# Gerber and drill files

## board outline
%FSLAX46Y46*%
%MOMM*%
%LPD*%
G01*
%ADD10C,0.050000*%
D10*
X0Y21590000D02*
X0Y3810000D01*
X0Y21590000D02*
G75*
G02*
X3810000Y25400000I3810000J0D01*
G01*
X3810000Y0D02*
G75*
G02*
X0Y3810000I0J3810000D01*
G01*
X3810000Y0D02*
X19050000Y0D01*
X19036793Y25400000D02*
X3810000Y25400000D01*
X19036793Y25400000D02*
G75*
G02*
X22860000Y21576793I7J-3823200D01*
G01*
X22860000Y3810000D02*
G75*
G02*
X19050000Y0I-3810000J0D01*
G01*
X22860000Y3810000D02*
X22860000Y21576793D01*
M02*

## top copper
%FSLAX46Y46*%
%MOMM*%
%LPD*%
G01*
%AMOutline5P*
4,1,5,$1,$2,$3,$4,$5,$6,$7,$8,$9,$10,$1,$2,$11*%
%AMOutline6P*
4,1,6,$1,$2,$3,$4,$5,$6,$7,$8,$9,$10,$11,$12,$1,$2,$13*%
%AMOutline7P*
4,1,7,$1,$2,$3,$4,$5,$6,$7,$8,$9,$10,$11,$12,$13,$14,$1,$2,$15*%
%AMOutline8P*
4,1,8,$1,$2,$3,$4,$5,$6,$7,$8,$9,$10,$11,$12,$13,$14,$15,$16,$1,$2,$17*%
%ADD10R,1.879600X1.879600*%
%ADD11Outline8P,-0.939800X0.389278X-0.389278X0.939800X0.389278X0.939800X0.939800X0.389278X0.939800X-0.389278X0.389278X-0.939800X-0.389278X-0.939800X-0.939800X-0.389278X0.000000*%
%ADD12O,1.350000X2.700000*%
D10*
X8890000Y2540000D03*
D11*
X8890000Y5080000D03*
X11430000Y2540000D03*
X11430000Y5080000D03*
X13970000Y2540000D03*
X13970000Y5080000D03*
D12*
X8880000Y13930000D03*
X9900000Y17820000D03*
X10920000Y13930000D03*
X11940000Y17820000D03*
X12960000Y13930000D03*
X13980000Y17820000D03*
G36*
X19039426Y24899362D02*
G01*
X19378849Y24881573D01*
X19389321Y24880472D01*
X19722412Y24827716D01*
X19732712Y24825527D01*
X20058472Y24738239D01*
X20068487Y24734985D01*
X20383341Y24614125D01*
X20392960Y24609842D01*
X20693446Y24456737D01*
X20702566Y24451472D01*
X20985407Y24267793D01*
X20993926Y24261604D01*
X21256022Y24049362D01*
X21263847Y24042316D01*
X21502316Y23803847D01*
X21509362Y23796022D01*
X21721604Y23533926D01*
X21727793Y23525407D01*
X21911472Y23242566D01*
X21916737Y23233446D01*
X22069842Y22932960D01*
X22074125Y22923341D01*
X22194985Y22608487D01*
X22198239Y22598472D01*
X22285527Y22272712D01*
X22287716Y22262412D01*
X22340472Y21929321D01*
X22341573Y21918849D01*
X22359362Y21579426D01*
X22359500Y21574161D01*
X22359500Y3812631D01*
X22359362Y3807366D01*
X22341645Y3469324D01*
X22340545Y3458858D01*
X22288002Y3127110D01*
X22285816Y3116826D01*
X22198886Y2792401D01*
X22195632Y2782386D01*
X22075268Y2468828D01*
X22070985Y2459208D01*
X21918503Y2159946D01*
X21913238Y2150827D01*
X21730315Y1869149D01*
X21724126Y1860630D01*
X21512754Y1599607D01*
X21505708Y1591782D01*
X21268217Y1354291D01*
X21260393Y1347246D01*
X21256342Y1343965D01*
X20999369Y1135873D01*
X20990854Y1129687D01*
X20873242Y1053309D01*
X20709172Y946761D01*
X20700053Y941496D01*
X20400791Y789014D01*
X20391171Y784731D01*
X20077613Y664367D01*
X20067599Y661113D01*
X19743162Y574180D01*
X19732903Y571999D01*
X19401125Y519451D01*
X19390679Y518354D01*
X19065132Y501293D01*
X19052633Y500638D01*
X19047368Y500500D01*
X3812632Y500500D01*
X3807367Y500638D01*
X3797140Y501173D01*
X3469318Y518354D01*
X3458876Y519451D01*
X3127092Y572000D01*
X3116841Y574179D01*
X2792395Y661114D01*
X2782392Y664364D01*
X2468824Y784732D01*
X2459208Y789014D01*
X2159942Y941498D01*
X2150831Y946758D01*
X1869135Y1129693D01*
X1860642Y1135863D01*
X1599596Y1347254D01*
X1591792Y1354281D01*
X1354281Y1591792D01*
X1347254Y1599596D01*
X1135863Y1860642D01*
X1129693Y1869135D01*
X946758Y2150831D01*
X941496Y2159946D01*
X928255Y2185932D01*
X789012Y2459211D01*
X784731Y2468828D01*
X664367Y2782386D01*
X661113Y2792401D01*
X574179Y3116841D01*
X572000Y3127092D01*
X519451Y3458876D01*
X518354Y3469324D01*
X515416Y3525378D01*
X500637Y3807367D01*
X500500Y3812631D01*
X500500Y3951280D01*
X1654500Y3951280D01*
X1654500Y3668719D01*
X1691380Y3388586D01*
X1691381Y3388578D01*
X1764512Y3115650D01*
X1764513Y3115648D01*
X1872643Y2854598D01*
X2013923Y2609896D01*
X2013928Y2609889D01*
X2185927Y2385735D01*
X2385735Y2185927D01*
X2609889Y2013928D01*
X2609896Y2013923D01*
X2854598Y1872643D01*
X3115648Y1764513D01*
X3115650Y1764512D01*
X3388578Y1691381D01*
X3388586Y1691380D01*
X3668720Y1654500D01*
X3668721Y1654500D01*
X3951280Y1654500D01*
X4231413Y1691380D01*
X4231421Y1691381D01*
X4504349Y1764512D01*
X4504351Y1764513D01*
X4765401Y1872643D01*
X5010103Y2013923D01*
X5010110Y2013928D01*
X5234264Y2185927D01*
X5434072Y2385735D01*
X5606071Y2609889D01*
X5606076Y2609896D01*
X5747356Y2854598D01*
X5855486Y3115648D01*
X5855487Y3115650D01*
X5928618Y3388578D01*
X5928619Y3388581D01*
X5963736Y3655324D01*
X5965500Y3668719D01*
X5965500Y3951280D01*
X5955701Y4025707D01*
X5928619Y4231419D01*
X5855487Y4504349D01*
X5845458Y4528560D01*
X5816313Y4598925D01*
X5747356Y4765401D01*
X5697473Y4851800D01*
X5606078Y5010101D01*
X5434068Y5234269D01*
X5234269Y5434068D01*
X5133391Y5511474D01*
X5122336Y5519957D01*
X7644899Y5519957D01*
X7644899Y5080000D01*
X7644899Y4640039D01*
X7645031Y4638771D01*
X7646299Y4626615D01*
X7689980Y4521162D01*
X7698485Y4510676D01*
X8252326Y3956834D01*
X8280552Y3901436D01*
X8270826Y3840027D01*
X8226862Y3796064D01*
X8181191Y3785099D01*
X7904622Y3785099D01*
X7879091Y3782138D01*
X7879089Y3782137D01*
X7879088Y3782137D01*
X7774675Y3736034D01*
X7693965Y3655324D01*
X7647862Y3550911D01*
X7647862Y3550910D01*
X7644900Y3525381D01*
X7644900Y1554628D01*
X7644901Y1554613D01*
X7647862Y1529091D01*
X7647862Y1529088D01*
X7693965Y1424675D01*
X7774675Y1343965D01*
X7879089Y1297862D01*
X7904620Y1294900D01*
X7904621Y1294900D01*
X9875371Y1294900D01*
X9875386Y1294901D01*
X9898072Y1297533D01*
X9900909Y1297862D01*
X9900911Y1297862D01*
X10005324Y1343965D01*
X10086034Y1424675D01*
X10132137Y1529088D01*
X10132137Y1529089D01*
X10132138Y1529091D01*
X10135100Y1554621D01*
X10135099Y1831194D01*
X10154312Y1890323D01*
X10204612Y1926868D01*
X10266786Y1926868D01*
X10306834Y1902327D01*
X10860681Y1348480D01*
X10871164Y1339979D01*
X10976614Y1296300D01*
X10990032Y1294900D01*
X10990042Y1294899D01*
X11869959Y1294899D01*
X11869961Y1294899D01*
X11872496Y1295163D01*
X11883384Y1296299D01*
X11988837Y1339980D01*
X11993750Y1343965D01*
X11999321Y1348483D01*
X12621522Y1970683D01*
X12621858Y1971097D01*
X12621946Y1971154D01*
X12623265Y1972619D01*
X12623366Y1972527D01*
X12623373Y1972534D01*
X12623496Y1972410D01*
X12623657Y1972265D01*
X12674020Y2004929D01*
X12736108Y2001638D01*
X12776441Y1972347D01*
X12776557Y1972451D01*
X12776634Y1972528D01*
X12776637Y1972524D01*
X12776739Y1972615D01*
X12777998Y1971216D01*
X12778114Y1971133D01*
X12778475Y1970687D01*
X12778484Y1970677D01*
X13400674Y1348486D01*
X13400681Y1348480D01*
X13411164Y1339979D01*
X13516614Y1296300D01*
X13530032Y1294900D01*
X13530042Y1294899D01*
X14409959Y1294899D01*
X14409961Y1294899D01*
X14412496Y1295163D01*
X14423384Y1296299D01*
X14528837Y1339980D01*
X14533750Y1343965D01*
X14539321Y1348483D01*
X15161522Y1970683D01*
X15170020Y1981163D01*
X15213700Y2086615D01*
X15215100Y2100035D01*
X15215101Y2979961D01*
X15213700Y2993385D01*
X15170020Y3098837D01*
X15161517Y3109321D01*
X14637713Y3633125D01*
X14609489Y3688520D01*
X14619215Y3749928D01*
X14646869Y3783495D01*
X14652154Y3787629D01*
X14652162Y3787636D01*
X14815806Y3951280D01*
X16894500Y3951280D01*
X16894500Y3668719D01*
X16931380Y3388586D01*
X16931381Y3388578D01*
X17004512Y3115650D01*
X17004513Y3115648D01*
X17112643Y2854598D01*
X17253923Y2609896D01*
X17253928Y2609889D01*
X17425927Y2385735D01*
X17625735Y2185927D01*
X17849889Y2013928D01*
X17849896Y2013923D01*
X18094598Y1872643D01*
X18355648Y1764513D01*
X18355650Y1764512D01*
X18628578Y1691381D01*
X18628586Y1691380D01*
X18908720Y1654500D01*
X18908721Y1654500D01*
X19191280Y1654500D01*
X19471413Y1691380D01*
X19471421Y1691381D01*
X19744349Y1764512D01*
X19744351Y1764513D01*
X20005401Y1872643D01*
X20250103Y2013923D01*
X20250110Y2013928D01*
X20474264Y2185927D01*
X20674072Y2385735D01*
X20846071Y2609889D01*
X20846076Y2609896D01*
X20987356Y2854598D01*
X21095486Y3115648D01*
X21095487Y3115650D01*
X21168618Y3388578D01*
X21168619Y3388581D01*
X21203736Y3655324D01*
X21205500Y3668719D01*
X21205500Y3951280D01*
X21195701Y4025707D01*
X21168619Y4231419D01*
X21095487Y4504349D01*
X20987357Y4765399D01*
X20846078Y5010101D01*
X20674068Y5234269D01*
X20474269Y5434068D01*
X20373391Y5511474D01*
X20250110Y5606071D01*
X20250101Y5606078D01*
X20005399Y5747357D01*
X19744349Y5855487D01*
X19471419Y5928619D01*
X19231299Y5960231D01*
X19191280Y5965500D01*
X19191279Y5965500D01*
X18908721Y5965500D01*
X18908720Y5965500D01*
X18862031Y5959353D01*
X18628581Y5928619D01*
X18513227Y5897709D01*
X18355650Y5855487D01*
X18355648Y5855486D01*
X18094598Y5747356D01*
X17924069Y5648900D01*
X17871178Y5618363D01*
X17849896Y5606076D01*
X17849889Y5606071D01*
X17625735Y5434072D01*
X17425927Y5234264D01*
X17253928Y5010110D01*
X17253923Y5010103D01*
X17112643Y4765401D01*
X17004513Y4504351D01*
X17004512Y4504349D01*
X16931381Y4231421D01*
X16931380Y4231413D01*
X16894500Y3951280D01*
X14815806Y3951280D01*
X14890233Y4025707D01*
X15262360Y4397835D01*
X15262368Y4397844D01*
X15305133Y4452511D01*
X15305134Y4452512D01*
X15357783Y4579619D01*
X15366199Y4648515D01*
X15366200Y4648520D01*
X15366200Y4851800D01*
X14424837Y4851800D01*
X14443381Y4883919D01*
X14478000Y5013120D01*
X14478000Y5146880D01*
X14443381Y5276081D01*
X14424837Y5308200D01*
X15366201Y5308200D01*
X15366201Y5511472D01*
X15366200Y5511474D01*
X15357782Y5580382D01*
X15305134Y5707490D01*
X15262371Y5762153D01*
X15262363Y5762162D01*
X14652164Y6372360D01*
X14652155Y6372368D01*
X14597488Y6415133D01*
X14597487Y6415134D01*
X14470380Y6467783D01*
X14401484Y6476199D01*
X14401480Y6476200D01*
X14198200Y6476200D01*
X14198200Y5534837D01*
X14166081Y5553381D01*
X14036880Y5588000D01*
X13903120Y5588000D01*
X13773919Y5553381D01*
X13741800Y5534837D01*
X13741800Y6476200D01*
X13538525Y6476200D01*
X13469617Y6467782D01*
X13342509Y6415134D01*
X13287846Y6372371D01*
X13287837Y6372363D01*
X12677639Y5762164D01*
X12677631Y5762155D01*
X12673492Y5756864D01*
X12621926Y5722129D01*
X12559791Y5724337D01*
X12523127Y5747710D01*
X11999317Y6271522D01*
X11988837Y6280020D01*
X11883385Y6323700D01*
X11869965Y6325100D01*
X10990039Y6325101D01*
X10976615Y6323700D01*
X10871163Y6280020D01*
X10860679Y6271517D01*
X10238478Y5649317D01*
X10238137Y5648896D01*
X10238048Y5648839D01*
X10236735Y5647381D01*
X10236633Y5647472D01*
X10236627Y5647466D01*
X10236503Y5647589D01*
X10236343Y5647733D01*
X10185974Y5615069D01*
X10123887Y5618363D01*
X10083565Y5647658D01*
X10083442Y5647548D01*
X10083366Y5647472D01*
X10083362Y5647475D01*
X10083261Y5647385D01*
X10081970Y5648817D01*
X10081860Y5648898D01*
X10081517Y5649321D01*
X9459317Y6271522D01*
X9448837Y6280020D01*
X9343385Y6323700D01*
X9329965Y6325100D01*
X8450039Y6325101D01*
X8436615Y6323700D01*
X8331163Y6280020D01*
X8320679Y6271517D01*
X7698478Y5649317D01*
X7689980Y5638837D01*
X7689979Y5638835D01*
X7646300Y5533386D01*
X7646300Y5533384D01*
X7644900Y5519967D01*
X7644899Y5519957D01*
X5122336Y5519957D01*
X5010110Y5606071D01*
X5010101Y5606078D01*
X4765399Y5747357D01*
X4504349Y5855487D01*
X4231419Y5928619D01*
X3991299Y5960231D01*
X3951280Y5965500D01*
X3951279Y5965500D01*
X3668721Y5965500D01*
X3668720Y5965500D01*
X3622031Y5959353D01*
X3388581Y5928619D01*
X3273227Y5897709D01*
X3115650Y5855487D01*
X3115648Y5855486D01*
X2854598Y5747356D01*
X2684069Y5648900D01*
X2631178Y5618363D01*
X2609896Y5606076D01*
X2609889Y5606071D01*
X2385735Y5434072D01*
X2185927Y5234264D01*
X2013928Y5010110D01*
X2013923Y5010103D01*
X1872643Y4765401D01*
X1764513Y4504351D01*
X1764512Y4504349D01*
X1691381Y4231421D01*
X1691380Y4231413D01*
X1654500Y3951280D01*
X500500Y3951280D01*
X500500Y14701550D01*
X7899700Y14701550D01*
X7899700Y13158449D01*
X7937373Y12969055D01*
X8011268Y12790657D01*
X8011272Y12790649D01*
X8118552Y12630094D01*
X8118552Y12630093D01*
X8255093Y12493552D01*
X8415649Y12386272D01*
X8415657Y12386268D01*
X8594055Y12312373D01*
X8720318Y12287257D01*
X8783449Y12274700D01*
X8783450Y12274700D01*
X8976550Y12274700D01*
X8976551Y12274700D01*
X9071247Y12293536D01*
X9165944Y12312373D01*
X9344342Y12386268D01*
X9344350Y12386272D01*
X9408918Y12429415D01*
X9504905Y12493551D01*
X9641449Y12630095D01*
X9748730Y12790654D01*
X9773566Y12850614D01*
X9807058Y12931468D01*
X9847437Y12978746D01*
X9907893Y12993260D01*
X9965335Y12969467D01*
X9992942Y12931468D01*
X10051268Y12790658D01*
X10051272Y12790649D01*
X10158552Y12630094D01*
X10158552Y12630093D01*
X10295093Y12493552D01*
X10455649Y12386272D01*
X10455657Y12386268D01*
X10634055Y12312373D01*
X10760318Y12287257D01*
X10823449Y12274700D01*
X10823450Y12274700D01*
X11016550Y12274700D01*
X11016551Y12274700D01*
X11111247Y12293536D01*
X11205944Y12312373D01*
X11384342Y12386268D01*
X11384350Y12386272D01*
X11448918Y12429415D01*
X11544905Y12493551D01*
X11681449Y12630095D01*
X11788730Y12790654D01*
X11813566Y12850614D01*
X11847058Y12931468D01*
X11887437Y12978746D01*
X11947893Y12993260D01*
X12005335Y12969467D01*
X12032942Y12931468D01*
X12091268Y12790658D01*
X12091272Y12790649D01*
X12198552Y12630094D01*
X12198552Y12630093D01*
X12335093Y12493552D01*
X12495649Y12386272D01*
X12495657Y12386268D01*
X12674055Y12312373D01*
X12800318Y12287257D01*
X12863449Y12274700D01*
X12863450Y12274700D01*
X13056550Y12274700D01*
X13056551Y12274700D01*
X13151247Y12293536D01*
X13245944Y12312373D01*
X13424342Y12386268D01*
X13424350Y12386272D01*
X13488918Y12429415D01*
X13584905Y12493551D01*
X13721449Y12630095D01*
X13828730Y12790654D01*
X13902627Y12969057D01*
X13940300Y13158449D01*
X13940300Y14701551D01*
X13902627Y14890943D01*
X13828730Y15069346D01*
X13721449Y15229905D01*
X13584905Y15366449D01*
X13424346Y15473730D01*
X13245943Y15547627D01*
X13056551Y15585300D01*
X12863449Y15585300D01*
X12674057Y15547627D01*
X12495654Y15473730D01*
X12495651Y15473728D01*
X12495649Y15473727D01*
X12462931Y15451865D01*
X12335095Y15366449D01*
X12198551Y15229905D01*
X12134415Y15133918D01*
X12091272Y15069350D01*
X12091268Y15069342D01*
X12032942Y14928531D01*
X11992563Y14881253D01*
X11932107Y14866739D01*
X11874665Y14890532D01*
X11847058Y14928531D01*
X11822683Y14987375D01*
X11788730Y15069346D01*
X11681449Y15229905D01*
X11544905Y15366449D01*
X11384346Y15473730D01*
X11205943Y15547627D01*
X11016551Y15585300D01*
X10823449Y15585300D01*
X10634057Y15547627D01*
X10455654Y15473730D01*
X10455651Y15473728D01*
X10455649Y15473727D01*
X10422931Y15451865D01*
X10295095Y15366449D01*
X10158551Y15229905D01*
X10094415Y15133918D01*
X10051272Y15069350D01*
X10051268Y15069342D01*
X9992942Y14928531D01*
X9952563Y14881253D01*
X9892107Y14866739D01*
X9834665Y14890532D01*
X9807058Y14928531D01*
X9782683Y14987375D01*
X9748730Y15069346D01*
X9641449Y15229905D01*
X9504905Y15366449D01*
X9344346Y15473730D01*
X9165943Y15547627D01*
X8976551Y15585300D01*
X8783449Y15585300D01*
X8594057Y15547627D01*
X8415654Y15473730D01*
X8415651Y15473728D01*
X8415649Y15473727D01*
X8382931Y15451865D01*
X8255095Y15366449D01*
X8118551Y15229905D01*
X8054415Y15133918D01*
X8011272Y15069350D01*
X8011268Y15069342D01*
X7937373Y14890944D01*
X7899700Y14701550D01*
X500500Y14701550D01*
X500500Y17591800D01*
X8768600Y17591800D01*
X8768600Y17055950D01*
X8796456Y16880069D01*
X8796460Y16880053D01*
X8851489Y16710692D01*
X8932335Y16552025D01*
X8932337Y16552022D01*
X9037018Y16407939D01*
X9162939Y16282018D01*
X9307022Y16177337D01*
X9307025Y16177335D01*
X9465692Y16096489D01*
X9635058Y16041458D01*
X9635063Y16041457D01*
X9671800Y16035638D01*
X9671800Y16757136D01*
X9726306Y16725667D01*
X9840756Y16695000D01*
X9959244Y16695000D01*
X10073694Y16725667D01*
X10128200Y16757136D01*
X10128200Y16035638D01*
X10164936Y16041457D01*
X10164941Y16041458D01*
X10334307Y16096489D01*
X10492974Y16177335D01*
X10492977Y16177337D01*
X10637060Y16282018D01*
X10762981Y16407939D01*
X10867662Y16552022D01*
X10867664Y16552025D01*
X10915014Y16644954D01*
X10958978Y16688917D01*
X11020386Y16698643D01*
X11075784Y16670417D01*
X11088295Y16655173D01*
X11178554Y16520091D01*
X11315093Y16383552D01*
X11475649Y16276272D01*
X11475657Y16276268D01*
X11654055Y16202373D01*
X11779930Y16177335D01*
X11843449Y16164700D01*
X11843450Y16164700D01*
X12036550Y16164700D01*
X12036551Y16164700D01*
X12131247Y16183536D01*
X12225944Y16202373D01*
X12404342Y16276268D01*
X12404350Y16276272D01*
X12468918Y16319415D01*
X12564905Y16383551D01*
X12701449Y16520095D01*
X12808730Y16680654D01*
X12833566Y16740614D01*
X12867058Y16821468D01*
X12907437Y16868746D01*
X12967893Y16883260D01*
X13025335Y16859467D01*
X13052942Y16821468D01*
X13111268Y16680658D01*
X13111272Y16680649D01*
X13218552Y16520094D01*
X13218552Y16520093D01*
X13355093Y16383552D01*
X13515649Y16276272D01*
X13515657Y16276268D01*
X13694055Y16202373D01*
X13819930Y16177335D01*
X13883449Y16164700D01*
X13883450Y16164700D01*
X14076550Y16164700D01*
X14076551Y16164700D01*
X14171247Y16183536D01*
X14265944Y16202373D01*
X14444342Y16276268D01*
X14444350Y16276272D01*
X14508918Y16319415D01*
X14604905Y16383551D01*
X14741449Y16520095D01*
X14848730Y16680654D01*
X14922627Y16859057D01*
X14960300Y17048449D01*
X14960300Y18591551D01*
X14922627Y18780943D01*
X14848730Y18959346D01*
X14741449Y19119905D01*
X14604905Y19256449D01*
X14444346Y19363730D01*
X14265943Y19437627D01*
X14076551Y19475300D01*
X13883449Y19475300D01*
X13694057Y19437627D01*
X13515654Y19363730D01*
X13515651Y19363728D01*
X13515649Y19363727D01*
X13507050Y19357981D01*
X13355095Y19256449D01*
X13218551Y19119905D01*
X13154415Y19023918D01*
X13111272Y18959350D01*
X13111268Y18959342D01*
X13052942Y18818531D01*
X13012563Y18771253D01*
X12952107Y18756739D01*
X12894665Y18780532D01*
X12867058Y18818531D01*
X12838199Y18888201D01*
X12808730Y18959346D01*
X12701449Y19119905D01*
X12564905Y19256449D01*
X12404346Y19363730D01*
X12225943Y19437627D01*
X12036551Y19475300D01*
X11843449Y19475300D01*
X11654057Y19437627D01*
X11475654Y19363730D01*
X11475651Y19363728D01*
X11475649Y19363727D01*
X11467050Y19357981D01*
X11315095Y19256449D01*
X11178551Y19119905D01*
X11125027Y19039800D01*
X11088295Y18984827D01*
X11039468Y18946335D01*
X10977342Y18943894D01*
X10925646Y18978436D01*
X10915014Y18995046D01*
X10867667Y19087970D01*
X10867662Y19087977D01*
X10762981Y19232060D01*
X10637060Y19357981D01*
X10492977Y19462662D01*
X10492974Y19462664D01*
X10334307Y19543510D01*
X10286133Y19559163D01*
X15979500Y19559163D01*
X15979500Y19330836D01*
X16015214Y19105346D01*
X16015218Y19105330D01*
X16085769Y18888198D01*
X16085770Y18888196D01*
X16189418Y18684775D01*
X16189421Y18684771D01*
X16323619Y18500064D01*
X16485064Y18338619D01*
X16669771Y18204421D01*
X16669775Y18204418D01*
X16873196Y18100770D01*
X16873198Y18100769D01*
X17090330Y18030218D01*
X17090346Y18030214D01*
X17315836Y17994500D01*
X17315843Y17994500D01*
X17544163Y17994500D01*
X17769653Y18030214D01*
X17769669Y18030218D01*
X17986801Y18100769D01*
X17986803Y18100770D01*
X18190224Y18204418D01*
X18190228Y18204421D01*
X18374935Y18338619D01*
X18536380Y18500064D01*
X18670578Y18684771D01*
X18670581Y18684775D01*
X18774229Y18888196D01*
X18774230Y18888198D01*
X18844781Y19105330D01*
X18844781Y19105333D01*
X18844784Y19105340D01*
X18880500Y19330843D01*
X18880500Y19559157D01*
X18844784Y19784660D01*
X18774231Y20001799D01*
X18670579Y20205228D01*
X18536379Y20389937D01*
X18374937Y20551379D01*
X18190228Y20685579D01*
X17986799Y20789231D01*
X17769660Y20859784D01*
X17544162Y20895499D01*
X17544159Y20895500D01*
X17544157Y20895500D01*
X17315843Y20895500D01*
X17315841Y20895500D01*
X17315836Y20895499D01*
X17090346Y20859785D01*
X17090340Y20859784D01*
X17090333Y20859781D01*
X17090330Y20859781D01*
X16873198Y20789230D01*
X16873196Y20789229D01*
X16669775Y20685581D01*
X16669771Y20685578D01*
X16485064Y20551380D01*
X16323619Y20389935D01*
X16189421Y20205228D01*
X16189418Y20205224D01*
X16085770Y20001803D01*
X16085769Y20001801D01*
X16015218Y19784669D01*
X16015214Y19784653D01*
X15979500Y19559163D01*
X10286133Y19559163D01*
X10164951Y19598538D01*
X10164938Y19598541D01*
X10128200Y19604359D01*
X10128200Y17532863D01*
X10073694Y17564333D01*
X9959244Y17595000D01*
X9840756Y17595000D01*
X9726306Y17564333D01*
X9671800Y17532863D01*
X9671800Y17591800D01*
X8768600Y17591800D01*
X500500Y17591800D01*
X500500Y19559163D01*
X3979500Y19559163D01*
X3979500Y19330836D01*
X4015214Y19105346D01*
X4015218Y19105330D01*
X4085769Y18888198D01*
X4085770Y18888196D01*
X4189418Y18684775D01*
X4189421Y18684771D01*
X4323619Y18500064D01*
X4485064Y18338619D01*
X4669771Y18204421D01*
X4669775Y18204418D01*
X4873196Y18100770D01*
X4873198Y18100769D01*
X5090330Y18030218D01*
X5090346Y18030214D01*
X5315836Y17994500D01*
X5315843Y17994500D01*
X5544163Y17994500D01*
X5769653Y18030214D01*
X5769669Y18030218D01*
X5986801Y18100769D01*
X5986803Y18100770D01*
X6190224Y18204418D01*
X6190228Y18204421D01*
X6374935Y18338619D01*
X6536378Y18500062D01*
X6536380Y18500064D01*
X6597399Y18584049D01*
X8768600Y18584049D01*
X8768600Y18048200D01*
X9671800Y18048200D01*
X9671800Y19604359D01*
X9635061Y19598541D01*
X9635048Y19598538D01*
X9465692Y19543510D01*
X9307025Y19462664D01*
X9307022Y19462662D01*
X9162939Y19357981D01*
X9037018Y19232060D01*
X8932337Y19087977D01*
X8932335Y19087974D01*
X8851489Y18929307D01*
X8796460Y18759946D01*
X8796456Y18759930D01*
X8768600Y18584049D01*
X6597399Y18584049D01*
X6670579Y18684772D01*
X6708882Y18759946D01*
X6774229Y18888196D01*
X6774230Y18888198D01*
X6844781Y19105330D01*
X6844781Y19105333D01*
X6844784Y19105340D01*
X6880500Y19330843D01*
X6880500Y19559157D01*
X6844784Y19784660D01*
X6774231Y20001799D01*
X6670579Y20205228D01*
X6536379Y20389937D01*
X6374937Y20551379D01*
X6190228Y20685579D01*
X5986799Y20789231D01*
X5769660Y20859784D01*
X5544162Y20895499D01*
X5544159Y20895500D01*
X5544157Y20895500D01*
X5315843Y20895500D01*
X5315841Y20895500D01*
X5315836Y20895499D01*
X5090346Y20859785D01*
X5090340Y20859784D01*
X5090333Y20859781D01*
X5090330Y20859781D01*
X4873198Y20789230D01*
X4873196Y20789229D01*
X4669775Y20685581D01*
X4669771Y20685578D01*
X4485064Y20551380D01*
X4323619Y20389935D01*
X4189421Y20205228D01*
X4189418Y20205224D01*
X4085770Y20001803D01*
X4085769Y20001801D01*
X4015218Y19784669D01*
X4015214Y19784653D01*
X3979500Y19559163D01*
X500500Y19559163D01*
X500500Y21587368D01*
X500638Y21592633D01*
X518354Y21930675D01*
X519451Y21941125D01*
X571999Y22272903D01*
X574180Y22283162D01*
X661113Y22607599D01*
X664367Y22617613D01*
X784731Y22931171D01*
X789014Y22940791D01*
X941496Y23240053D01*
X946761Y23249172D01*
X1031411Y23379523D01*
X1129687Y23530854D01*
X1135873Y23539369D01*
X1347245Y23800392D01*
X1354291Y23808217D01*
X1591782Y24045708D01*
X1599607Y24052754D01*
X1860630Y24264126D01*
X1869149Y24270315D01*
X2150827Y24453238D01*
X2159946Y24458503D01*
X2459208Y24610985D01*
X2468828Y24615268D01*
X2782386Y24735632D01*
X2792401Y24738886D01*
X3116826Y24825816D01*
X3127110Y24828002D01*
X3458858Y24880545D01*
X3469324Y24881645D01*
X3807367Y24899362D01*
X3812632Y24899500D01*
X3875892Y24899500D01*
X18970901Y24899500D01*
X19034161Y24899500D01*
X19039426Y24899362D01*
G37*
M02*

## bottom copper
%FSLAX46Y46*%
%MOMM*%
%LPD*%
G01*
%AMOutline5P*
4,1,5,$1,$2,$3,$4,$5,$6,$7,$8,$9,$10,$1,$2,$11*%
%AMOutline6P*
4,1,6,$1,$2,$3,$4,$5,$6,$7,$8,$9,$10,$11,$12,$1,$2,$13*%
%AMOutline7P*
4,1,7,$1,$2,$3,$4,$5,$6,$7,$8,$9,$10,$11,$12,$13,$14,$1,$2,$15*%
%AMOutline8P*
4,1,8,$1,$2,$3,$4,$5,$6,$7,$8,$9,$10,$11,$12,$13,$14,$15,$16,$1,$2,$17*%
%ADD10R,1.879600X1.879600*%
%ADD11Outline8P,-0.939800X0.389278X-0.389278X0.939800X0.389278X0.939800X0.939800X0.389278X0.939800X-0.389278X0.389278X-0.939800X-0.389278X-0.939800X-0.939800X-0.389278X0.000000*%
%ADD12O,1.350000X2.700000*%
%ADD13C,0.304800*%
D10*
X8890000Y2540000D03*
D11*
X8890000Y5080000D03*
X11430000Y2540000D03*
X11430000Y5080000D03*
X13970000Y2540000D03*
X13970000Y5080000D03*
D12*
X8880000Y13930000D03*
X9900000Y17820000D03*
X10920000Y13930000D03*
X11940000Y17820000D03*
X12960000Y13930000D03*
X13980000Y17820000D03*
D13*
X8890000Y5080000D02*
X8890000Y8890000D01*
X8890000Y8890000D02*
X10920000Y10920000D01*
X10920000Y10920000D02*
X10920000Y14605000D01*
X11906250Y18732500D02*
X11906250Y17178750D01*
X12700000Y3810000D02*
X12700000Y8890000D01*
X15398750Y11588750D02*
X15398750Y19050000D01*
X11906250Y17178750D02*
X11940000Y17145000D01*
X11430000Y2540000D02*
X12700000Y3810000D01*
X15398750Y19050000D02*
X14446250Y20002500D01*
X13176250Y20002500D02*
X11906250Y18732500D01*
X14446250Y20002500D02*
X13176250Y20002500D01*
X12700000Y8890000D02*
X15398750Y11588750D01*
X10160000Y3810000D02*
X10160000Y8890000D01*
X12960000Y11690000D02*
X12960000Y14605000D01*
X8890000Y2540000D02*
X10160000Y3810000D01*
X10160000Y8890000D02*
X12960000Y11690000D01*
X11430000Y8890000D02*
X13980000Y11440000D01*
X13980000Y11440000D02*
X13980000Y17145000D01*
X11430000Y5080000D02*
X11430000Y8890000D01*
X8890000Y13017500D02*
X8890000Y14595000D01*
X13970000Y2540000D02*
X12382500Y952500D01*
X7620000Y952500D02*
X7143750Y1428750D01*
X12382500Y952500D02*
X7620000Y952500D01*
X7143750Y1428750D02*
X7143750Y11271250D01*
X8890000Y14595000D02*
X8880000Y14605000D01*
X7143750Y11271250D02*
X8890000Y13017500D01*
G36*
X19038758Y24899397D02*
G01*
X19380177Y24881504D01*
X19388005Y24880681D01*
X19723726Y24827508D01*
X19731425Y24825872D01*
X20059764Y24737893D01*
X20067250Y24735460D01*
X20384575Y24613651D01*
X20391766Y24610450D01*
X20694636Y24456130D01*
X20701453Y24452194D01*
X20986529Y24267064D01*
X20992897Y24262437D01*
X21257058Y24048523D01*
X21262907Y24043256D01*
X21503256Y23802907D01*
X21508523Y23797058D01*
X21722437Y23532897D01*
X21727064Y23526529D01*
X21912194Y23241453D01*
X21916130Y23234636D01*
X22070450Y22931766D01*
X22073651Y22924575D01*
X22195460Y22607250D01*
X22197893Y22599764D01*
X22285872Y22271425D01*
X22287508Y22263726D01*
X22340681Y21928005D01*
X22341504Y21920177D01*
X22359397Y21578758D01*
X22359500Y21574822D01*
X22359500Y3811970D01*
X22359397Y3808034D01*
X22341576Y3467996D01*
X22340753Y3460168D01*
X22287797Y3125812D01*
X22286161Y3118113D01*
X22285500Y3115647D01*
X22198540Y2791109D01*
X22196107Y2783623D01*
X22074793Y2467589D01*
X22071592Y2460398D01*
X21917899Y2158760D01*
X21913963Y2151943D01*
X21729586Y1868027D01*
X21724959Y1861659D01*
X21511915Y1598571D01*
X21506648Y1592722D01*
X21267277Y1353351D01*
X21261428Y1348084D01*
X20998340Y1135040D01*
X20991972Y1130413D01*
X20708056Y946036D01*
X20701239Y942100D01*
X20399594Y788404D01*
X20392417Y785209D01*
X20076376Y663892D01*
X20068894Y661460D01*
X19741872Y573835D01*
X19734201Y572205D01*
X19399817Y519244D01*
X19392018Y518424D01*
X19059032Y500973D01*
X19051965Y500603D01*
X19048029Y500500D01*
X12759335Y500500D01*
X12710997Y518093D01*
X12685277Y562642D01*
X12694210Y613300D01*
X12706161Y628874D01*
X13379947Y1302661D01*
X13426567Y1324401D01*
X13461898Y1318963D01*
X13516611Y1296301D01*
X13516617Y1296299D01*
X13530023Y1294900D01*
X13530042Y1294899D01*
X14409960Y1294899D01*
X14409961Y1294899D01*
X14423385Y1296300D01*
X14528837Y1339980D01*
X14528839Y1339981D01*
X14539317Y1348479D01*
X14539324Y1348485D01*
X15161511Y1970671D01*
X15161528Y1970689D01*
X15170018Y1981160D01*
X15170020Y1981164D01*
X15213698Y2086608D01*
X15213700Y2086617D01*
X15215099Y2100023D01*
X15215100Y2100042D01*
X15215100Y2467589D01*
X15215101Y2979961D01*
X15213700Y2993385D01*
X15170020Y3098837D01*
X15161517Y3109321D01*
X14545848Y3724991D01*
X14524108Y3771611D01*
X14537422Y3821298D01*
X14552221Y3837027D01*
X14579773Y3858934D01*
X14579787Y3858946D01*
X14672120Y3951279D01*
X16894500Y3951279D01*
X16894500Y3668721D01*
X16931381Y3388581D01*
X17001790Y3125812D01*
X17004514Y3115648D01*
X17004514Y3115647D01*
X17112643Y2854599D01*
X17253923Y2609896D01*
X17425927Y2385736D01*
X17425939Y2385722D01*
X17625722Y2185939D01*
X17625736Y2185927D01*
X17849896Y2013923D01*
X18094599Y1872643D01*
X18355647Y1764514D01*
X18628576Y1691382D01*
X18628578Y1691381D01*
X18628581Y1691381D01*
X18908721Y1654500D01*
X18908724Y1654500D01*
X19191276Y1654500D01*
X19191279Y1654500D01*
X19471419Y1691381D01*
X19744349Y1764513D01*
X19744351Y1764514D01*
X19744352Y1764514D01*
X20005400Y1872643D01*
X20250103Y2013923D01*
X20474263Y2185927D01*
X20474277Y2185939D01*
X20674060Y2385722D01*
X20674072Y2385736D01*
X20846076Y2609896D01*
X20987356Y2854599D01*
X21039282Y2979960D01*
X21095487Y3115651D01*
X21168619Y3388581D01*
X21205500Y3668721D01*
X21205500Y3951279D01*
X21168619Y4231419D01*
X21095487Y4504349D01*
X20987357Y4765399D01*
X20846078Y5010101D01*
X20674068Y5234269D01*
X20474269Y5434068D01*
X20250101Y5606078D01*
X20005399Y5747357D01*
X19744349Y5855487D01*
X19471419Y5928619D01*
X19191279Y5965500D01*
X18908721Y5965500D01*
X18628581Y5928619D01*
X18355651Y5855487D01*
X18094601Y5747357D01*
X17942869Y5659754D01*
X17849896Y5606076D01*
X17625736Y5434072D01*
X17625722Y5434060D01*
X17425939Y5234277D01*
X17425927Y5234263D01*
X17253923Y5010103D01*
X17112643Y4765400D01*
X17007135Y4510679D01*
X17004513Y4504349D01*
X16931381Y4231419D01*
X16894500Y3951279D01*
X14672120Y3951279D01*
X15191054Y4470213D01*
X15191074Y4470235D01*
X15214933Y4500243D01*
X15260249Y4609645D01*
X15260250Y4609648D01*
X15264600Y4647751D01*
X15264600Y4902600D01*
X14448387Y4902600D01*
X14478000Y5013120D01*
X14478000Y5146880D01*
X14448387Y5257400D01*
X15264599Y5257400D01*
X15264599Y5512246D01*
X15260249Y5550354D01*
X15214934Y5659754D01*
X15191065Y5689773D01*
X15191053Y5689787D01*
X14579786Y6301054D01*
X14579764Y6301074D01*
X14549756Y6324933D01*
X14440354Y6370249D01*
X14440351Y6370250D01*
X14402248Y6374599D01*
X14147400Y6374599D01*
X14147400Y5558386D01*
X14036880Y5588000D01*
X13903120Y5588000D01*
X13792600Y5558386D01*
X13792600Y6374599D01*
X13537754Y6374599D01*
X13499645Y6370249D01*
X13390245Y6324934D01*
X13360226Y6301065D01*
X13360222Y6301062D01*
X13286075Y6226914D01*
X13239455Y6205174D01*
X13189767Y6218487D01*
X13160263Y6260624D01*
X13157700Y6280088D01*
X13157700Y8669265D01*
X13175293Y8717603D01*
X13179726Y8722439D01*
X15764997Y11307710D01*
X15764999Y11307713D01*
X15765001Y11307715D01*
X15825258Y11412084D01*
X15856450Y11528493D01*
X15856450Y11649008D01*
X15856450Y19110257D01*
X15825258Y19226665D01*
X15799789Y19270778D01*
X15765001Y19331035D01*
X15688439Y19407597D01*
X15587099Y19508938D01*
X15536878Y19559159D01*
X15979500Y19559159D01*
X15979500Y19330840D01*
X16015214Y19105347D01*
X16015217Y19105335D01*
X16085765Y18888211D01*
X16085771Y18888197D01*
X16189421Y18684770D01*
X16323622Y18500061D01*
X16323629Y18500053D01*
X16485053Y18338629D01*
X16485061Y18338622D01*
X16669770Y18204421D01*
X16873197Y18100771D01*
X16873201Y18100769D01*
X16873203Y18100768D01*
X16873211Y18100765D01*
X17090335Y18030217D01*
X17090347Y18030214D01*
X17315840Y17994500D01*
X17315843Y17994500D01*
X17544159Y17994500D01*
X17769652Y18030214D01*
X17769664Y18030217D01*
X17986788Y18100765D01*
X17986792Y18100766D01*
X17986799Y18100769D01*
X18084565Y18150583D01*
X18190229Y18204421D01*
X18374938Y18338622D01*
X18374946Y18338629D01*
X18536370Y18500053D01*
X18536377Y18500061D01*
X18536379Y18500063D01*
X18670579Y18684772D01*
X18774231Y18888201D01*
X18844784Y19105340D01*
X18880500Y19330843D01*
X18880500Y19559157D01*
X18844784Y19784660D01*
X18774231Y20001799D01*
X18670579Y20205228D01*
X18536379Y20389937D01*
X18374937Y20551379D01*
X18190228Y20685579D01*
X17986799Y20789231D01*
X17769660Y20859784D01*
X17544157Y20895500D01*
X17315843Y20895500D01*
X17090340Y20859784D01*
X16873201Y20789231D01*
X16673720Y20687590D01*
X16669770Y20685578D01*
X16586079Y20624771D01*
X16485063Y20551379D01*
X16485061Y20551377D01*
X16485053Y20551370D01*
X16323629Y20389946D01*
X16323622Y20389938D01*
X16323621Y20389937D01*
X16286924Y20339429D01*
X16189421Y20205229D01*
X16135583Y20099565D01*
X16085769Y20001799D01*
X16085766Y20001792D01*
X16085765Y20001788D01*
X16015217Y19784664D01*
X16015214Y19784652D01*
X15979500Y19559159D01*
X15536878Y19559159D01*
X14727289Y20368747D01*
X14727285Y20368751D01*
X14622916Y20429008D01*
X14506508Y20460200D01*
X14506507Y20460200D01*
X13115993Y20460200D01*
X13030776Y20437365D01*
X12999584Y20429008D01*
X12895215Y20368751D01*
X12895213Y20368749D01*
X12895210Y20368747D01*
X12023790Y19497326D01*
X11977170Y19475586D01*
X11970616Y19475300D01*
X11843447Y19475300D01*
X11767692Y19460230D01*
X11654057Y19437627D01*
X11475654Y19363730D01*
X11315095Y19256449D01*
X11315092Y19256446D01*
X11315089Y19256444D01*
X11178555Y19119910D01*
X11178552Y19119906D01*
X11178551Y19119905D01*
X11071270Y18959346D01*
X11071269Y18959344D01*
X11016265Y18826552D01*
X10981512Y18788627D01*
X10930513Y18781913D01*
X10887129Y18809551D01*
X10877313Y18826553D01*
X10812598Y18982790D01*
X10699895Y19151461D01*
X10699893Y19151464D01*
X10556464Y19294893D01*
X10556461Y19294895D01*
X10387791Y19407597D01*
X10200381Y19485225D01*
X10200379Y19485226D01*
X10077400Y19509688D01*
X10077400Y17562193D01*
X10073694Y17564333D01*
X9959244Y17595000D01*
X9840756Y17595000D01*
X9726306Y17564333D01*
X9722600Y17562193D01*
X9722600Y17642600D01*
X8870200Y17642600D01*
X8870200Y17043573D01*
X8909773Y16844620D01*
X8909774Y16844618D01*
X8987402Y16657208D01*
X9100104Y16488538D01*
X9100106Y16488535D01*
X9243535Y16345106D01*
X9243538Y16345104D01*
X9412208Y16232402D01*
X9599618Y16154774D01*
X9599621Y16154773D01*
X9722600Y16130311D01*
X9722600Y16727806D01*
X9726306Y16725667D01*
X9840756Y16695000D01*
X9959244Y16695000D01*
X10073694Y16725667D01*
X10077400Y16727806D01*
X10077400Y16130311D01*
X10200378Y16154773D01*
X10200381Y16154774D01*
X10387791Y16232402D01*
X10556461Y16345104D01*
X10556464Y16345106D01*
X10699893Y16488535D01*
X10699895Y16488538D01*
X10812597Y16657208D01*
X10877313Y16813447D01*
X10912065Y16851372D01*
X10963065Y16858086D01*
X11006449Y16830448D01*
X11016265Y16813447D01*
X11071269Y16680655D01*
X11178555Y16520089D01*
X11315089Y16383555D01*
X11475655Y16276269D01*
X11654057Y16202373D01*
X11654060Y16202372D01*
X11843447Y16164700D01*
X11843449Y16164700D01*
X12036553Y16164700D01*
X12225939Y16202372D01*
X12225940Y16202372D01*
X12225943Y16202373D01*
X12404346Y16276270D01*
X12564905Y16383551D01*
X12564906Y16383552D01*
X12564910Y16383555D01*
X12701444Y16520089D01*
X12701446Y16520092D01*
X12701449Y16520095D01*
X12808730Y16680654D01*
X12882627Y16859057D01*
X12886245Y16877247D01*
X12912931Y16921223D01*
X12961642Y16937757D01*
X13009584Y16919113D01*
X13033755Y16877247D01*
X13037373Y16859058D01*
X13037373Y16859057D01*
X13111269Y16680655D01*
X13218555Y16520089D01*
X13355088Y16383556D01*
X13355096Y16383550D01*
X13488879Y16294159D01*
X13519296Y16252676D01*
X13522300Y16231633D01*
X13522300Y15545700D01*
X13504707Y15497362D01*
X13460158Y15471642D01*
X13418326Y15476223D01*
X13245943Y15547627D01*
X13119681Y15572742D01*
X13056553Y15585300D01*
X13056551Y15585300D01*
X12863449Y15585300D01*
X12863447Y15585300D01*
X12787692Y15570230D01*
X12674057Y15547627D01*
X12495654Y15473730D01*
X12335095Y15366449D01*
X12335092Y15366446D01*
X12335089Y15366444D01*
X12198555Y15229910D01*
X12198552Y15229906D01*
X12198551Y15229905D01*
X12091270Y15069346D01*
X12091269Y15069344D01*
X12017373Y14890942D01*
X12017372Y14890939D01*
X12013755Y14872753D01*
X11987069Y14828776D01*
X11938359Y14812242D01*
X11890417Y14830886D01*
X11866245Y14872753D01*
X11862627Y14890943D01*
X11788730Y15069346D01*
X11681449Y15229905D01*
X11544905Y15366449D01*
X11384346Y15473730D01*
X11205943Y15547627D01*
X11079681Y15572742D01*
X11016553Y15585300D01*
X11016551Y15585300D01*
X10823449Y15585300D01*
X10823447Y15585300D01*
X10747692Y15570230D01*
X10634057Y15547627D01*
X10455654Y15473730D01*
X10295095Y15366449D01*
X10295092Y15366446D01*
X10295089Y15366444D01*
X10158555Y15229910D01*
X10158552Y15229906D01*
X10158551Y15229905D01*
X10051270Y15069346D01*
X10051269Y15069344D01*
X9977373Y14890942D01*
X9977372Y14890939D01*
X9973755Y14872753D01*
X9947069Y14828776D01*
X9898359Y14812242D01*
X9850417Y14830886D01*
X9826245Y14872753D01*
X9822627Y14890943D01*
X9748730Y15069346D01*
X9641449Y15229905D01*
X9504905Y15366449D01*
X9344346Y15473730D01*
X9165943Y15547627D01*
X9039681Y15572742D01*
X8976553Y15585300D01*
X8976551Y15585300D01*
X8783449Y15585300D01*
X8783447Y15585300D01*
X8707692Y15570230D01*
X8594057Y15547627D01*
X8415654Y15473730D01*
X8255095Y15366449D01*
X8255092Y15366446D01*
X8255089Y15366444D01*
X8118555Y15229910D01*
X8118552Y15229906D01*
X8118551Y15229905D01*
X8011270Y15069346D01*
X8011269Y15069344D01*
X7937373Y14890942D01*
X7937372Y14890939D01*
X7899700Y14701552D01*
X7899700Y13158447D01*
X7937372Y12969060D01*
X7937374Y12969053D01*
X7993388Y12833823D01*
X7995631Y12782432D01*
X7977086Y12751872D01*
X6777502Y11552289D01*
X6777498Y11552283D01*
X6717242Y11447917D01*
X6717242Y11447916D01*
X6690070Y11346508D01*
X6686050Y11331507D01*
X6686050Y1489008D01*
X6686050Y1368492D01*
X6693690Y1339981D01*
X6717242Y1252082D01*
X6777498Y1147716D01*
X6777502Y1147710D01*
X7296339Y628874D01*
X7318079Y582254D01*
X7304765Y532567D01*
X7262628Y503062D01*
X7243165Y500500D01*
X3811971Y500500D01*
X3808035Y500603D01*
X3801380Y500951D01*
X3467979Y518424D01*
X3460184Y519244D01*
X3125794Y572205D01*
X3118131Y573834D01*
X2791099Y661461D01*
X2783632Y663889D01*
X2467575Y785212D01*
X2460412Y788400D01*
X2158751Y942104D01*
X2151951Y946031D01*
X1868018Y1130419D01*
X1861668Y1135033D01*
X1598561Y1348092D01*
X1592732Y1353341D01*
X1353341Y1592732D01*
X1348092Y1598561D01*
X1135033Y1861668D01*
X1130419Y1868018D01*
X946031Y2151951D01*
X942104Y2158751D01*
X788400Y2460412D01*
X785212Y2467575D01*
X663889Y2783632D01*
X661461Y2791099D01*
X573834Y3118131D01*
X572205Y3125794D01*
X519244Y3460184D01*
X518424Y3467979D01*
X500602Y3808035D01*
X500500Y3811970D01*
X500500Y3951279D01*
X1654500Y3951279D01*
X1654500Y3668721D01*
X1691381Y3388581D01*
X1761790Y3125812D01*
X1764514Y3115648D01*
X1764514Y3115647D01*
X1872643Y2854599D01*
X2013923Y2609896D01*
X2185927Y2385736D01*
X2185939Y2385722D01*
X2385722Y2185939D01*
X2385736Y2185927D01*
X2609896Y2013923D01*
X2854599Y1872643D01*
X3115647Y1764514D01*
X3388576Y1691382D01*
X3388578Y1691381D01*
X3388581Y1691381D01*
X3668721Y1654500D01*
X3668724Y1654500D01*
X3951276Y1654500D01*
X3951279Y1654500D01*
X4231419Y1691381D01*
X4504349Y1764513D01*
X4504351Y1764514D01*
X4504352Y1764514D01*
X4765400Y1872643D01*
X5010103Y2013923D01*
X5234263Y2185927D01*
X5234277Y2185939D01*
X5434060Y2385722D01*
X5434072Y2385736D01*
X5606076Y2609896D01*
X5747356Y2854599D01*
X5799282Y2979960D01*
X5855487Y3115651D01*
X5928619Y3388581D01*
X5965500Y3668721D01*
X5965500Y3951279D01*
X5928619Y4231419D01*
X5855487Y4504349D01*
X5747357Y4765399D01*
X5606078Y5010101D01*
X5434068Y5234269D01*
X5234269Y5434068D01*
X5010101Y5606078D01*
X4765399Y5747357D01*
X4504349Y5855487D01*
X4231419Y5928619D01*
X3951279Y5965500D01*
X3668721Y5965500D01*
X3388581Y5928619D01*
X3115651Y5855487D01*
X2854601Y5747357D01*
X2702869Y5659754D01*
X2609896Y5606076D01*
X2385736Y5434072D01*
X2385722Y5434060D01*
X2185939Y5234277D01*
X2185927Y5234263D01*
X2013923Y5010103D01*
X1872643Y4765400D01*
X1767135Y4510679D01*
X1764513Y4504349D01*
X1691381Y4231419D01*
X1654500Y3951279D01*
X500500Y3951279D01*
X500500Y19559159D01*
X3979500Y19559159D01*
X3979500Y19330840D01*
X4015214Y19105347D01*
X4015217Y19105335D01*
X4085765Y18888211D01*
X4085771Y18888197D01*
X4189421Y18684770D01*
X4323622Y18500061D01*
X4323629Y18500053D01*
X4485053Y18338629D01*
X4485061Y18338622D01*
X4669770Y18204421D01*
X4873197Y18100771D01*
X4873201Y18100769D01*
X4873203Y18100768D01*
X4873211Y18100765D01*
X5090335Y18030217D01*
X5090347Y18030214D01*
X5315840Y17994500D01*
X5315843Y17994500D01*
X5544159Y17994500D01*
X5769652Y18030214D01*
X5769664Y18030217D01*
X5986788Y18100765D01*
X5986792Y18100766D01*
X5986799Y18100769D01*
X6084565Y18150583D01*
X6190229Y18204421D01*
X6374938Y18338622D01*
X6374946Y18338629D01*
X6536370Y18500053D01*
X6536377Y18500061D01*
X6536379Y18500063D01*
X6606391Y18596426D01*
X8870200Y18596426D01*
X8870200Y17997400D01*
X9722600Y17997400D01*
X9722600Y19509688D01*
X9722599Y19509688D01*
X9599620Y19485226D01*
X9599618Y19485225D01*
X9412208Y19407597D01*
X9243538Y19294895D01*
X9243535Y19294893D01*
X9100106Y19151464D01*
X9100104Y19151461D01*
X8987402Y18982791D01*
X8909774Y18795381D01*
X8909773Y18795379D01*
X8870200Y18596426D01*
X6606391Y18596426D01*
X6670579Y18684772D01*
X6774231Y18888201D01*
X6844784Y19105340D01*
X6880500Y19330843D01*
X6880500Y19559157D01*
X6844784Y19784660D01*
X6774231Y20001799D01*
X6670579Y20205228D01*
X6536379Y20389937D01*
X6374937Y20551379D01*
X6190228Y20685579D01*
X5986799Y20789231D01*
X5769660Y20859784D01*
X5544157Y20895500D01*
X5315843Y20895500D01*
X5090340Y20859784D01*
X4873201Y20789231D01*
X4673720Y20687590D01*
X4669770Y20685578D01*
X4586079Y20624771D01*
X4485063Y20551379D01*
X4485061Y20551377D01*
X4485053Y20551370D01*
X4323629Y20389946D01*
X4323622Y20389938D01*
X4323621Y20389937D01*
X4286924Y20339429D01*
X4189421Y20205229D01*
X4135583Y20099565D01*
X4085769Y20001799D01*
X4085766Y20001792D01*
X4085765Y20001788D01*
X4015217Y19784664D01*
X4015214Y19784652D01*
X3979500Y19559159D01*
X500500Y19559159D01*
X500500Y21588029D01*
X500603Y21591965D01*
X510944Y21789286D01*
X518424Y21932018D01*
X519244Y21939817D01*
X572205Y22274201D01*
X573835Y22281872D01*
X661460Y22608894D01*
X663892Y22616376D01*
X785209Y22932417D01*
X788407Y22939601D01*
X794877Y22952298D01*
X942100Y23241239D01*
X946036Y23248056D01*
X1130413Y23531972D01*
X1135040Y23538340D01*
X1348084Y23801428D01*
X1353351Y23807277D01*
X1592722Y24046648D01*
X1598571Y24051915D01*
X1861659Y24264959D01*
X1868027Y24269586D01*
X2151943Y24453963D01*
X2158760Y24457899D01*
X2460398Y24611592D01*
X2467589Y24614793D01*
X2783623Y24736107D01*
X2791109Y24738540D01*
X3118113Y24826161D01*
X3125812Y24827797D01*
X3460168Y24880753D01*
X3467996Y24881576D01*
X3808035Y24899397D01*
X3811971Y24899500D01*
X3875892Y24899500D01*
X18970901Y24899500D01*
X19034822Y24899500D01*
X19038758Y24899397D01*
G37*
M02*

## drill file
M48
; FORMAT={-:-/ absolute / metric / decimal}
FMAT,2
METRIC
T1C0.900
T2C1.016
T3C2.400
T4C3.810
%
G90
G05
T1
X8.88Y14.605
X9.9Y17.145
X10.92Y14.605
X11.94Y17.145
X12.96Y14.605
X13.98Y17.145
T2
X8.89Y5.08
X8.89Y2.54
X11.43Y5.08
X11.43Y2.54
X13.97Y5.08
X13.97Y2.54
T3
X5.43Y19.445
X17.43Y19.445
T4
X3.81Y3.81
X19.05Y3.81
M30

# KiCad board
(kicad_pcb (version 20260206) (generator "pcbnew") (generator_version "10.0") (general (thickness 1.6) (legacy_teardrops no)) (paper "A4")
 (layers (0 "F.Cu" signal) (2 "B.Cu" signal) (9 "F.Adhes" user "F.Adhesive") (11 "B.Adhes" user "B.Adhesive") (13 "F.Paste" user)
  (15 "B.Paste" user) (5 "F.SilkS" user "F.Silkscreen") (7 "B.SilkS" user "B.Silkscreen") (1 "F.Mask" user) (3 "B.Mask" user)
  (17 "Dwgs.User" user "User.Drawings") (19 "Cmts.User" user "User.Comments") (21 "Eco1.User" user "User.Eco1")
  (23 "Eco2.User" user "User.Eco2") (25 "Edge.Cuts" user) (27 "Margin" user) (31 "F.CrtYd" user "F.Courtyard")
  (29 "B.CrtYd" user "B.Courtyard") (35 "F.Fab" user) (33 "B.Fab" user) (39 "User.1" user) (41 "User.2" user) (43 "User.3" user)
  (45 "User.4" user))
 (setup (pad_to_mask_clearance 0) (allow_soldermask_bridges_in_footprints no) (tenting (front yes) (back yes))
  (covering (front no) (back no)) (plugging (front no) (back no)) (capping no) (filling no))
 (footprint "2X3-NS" (layer "F.Cu") (at 11.43 -3.81)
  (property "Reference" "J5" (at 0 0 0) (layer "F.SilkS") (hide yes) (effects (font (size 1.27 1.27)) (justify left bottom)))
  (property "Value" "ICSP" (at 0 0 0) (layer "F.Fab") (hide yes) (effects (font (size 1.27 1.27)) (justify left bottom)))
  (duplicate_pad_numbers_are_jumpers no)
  (pad "1" thru_hole rect (at -2.54 1.27) (size 1.8796 1.8796) (drill 1.016) (layers "*.Cu" "*.Mask") (remove_unused_layers no) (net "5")
   (solder_mask_margin 0.0762) (thermal_bridge_angle 0))
  (pad "2" thru_hole roundrect (at -2.54 -1.27) (size 1.8796 1.8796) (drill 1.016) (layers "*.Cu" "*.Mask") (remove_unused_layers no)
   (roundrect_rratio 0.25) (chamfer_ratio 0.2928932188) (chamfer top_left top_right bottom_left bottom_right) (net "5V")
   (solder_mask_margin 0.0762) (thermal_bridge_angle 0))
  (pad "3" thru_hole roundrect (at 0 1.27) (size 1.8796 1.8796) (drill 1.016) (layers "*.Cu" "*.Mask") (remove_unused_layers no)
   (roundrect_rratio 0.25) (chamfer_ratio 0.2928932188) (chamfer top_left top_right bottom_left bottom_right) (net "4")
   (solder_mask_margin 0.0762) (thermal_bridge_angle 0))
  (pad "4" thru_hole roundrect (at 0 -1.27) (size 1.8796 1.8796) (drill 1.016) (layers "*.Cu" "*.Mask") (remove_unused_layers no)
   (roundrect_rratio 0.25) (chamfer_ratio 0.2928932188) (chamfer top_left top_right bottom_left bottom_right) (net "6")
   (solder_mask_margin 0.0762) (thermal_bridge_angle 0))
  (pad "5" thru_hole roundrect (at 2.54 1.27) (size 1.8796 1.8796) (drill 1.016) (layers "*.Cu" "*.Mask") (remove_unused_layers no)
   (roundrect_rratio 0.25) (chamfer_ratio 0.2928932188) (chamfer top_left top_right bottom_left bottom_right) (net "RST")
   (solder_mask_margin 0.0762) (thermal_bridge_angle 0))
  (pad "6" thru_hole roundrect (at 2.54 -1.27) (size 1.8796 1.8796) (drill 1.016) (layers "*.Cu" "*.Mask") (remove_unused_layers no)
   (roundrect_rratio 0.25) (chamfer_ratio 0.2928932188) (chamfer top_left top_right bottom_left bottom_right) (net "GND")
   (solder_mask_margin 0.0762) (thermal_bridge_angle 0)))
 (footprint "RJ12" (layer "F.Cu") (at 11.43 -17.145 180)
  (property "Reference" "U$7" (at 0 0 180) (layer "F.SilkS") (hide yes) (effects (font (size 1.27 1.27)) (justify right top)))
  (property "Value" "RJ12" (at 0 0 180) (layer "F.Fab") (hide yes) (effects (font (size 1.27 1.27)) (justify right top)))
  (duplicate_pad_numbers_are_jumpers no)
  (pad "" np_thru_hole circle (at -6 2.3 180) (size 2.4 2.4) (drill 2.4) (layers "*.Cu" "*.Mask"))
  (pad "" np_thru_hole circle (at 6 2.3 180) (size 2.4 2.4) (drill 2.4) (layers "*.Cu" "*.Mask"))
  (pad "1" thru_hole oval (at 2.55 -2.54 270) (size 2.7 1.35) (drill 0.9 (offset 0.675 0)) (layers "*.Cu" "*.Mask")
   (remove_unused_layers no) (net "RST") (solder_mask_margin 0.0762) (thermal_bridge_angle 0))
  (pad "2" thru_hole oval (at 1.53 0 90) (size 2.7 1.35) (drill 0.9 (offset 0.675 0)) (layers "*.Cu" "*.Mask") (remove_unused_layers no)
   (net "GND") (solder_mask_margin 0.0762) (thermal_bridge_angle 0))
  (pad "3" thru_hole oval (at 0.51 -2.54 270) (size 2.7 1.35) (drill 0.9 (offset 0.675 0)) (layers "*.Cu" "*.Mask")
   (remove_unused_layers no) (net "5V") (solder_mask_margin 0.0762) (thermal_bridge_angle 0))
  (pad "4" thru_hole oval (at -0.51 0 90) (size 2.7 1.35) (drill 0.9 (offset 0.675 0)) (layers "*.Cu" "*.Mask") (remove_unused_layers no)
   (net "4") (solder_mask_margin 0.0762) (thermal_bridge_angle 0))
  (pad "5" thru_hole oval (at -1.53 -2.54 270) (size 2.7 1.35) (drill 0.9 (offset 0.675 0)) (layers "*.Cu" "*.Mask")
   (remove_unused_layers no) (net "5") (solder_mask_margin 0.0762) (thermal_bridge_angle 0))
  (pad "6" thru_hole oval (at -2.55 0 90) (size 2.7 1.35) (drill 0.9 (offset 0.675 0)) (layers "*.Cu" "*.Mask") (remove_unused_layers no)
   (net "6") (solder_mask_margin 0.0762) (thermal_bridge_angle 0)))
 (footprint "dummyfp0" (layer "F.Cu") (at 3.81 -3.81)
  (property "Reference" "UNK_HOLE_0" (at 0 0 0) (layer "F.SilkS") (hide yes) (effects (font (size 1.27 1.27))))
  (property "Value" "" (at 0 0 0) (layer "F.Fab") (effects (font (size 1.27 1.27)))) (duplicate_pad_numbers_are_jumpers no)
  (pad "" np_thru_hole circle (at 0 0) (size 3.81 3.81) (drill 3.81) (layers "*.Cu" "*.Mask")))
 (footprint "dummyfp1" (layer "F.Cu") (at 19.05 -3.81)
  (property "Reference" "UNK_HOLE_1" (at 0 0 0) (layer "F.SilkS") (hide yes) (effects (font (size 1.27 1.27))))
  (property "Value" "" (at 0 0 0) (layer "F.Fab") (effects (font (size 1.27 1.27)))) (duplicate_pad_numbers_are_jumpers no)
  (pad "" np_thru_hole circle (at 0 0) (size 3.81 3.81) (drill 3.81) (layers "*.Cu" "*.Mask")))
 (gr_line (start 0 -21.59) (end 0 -3.81) (stroke (width 0.05) (type solid)) (layer "Edge.Cuts"))
 (gr_arc (start 0 -21.59) (mid 1.115923 -24.284077) (end 3.81 -25.4) (stroke (width 0.05) (type solid)) (layer "Edge.Cuts"))
 (gr_arc (start 3.81 0) (mid 1.115923 -1.115923) (end 0 -3.81) (stroke (width 0.05) (type solid)) (layer "Edge.Cuts"))
 (gr_line (start 3.81 0) (end 19.05 0) (stroke (width 0.05) (type solid)) (layer "Edge.Cuts"))
 (gr_line (start 19.036793 -25.4) (end 3.81 -25.4) (stroke (width 0.05) (type solid)) (layer "Edge.Cuts"))
 (gr_arc (start 19.036793 -25.4) (mid 21.740209 -24.280209) (end 22.86 -21.576793) (stroke (width 0.05) (type solid)) (layer "Edge.Cuts"))
 (gr_arc (start 22.86 -3.81) (mid 21.744077 -1.115923) (end 19.05 0) (stroke (width 0.05) (type solid)) (layer "Edge.Cuts"))
 (gr_line (start 22.86 -3.81) (end 22.86 -21.576793) (stroke (width 0.05) (type solid)) (layer "Edge.Cuts"))
 (segment (start 8.89 -5.08) (end 8.89 -8.89) (width 0.3048) (layer "B.Cu") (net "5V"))
 (segment (start 8.89 -8.89) (end 10.92 -10.92) (width 0.3048) (layer "B.Cu") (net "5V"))
 (segment (start 10.92 -10.92) (end 10.92 -14.605) (width 0.3048) (layer "B.Cu") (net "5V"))
 (segment (start 11.90625 -18.7325) (end 11.90625 -17.17875) (width 0.3048) (layer "B.Cu") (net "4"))
 (segment (start 12.7 -3.81) (end 12.7 -8.89) (width 0.3048) (layer "B.Cu") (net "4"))
 (segment (start 15.39875 -11.58875) (end 15.39875 -19.05) (width 0.3048) (layer "B.Cu") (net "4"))
 (segment (start 11.90625 -17.17875) (end 11.94 -17.145) (width 0.3048) (layer "B.Cu") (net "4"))
 (segment (start 11.43 -2.54) (end 12.7 -3.81) (width 0.3048) (layer "B.Cu") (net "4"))
 (segment (start 15.39875 -19.05) (end 14.44625 -20.0025) (width 0.3048) (layer "B.Cu") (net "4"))
 (segment (start 13.17625 -20.0025) (end 11.90625 -18.7325) (width 0.3048) (layer "B.Cu") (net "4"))
 (segment (start 14.44625 -20.0025) (end 13.17625 -20.0025) (width 0.3048) (layer "B.Cu") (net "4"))
 (segment (start 12.7 -8.89) (end 15.39875 -11.58875) (width 0.3048) (layer "B.Cu") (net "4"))
 (segment (start 10.16 -3.81) (end 10.16 -8.89) (width 0.3048) (layer "B.Cu") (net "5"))
 (segment (start 12.96 -11.69) (end 12.96 -14.605) (width 0.3048) (layer "B.Cu") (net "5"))
 (segment (start 8.89 -2.54) (end 10.16 -3.81) (width 0.3048) (layer "B.Cu") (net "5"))
 (segment (start 10.16 -8.89) (end 12.96 -11.69) (width 0.3048) (layer "B.Cu") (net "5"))
 (segment (start 11.43 -8.89) (end 13.98 -11.44) (width 0.3048) (layer "B.Cu") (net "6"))
 (segment (start 13.98 -11.44) (end 13.98 -17.145) (width 0.3048) (layer "B.Cu") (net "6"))
 (segment (start 11.43 -5.08) (end 11.43 -8.89) (width 0.3048) (layer "B.Cu") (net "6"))
 (segment (start 8.89 -13.0175) (end 8.89 -14.595) (width 0.3048) (layer "B.Cu") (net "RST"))
 (segment (start 13.97 -2.54) (end 12.3825 -0.9525) (width 0.3048) (layer "B.Cu") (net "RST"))
 (segment (start 7.62 -0.9525) (end 7.14375 -1.42875) (width 0.3048) (layer "B.Cu") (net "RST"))
 (segment (start 12.3825 -0.9525) (end 7.62 -0.9525) (width 0.3048) (layer "B.Cu") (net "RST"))
 (segment (start 7.14375 -1.42875) (end 7.14375 -11.27125) (width 0.3048) (layer "B.Cu") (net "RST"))
 (segment (start 8.89 -14.595) (end 8.88 -14.605) (width 0.3048) (layer "B.Cu") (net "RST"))
 (segment (start 7.14375 -11.27125) (end 8.89 -13.0175) (width 0.3048) (layer "B.Cu") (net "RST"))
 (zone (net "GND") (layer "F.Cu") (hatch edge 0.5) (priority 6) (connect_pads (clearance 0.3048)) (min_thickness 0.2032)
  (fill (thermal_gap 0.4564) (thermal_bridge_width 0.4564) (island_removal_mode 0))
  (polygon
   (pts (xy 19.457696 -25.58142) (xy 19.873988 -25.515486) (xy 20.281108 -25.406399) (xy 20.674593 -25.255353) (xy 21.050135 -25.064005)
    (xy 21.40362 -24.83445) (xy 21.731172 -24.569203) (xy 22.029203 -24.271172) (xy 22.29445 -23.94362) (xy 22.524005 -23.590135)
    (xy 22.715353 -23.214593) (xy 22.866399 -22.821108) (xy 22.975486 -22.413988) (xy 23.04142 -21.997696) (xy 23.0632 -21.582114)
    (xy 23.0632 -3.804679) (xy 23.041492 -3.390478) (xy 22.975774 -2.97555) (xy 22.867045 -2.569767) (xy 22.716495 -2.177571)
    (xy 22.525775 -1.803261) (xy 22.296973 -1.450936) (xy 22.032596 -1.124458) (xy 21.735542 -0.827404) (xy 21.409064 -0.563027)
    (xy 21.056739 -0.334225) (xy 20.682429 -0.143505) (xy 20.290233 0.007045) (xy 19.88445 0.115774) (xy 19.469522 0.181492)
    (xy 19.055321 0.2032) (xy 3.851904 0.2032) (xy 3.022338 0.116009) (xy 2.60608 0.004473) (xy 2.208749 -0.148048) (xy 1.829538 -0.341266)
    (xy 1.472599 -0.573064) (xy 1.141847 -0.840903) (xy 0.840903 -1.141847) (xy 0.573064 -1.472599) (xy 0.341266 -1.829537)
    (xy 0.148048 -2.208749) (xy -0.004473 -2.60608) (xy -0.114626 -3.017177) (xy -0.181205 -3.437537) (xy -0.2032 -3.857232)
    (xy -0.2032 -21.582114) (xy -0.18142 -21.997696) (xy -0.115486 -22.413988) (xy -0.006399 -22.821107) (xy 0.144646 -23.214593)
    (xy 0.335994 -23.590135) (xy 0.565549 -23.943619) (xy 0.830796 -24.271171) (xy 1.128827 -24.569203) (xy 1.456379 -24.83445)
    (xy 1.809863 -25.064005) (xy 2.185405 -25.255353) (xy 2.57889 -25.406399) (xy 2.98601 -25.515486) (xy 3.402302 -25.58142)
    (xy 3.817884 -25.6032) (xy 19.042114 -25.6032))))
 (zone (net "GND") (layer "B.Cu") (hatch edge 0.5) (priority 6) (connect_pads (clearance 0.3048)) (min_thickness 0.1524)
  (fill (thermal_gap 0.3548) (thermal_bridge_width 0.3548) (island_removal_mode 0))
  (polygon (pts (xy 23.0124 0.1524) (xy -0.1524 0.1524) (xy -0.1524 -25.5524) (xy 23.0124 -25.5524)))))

